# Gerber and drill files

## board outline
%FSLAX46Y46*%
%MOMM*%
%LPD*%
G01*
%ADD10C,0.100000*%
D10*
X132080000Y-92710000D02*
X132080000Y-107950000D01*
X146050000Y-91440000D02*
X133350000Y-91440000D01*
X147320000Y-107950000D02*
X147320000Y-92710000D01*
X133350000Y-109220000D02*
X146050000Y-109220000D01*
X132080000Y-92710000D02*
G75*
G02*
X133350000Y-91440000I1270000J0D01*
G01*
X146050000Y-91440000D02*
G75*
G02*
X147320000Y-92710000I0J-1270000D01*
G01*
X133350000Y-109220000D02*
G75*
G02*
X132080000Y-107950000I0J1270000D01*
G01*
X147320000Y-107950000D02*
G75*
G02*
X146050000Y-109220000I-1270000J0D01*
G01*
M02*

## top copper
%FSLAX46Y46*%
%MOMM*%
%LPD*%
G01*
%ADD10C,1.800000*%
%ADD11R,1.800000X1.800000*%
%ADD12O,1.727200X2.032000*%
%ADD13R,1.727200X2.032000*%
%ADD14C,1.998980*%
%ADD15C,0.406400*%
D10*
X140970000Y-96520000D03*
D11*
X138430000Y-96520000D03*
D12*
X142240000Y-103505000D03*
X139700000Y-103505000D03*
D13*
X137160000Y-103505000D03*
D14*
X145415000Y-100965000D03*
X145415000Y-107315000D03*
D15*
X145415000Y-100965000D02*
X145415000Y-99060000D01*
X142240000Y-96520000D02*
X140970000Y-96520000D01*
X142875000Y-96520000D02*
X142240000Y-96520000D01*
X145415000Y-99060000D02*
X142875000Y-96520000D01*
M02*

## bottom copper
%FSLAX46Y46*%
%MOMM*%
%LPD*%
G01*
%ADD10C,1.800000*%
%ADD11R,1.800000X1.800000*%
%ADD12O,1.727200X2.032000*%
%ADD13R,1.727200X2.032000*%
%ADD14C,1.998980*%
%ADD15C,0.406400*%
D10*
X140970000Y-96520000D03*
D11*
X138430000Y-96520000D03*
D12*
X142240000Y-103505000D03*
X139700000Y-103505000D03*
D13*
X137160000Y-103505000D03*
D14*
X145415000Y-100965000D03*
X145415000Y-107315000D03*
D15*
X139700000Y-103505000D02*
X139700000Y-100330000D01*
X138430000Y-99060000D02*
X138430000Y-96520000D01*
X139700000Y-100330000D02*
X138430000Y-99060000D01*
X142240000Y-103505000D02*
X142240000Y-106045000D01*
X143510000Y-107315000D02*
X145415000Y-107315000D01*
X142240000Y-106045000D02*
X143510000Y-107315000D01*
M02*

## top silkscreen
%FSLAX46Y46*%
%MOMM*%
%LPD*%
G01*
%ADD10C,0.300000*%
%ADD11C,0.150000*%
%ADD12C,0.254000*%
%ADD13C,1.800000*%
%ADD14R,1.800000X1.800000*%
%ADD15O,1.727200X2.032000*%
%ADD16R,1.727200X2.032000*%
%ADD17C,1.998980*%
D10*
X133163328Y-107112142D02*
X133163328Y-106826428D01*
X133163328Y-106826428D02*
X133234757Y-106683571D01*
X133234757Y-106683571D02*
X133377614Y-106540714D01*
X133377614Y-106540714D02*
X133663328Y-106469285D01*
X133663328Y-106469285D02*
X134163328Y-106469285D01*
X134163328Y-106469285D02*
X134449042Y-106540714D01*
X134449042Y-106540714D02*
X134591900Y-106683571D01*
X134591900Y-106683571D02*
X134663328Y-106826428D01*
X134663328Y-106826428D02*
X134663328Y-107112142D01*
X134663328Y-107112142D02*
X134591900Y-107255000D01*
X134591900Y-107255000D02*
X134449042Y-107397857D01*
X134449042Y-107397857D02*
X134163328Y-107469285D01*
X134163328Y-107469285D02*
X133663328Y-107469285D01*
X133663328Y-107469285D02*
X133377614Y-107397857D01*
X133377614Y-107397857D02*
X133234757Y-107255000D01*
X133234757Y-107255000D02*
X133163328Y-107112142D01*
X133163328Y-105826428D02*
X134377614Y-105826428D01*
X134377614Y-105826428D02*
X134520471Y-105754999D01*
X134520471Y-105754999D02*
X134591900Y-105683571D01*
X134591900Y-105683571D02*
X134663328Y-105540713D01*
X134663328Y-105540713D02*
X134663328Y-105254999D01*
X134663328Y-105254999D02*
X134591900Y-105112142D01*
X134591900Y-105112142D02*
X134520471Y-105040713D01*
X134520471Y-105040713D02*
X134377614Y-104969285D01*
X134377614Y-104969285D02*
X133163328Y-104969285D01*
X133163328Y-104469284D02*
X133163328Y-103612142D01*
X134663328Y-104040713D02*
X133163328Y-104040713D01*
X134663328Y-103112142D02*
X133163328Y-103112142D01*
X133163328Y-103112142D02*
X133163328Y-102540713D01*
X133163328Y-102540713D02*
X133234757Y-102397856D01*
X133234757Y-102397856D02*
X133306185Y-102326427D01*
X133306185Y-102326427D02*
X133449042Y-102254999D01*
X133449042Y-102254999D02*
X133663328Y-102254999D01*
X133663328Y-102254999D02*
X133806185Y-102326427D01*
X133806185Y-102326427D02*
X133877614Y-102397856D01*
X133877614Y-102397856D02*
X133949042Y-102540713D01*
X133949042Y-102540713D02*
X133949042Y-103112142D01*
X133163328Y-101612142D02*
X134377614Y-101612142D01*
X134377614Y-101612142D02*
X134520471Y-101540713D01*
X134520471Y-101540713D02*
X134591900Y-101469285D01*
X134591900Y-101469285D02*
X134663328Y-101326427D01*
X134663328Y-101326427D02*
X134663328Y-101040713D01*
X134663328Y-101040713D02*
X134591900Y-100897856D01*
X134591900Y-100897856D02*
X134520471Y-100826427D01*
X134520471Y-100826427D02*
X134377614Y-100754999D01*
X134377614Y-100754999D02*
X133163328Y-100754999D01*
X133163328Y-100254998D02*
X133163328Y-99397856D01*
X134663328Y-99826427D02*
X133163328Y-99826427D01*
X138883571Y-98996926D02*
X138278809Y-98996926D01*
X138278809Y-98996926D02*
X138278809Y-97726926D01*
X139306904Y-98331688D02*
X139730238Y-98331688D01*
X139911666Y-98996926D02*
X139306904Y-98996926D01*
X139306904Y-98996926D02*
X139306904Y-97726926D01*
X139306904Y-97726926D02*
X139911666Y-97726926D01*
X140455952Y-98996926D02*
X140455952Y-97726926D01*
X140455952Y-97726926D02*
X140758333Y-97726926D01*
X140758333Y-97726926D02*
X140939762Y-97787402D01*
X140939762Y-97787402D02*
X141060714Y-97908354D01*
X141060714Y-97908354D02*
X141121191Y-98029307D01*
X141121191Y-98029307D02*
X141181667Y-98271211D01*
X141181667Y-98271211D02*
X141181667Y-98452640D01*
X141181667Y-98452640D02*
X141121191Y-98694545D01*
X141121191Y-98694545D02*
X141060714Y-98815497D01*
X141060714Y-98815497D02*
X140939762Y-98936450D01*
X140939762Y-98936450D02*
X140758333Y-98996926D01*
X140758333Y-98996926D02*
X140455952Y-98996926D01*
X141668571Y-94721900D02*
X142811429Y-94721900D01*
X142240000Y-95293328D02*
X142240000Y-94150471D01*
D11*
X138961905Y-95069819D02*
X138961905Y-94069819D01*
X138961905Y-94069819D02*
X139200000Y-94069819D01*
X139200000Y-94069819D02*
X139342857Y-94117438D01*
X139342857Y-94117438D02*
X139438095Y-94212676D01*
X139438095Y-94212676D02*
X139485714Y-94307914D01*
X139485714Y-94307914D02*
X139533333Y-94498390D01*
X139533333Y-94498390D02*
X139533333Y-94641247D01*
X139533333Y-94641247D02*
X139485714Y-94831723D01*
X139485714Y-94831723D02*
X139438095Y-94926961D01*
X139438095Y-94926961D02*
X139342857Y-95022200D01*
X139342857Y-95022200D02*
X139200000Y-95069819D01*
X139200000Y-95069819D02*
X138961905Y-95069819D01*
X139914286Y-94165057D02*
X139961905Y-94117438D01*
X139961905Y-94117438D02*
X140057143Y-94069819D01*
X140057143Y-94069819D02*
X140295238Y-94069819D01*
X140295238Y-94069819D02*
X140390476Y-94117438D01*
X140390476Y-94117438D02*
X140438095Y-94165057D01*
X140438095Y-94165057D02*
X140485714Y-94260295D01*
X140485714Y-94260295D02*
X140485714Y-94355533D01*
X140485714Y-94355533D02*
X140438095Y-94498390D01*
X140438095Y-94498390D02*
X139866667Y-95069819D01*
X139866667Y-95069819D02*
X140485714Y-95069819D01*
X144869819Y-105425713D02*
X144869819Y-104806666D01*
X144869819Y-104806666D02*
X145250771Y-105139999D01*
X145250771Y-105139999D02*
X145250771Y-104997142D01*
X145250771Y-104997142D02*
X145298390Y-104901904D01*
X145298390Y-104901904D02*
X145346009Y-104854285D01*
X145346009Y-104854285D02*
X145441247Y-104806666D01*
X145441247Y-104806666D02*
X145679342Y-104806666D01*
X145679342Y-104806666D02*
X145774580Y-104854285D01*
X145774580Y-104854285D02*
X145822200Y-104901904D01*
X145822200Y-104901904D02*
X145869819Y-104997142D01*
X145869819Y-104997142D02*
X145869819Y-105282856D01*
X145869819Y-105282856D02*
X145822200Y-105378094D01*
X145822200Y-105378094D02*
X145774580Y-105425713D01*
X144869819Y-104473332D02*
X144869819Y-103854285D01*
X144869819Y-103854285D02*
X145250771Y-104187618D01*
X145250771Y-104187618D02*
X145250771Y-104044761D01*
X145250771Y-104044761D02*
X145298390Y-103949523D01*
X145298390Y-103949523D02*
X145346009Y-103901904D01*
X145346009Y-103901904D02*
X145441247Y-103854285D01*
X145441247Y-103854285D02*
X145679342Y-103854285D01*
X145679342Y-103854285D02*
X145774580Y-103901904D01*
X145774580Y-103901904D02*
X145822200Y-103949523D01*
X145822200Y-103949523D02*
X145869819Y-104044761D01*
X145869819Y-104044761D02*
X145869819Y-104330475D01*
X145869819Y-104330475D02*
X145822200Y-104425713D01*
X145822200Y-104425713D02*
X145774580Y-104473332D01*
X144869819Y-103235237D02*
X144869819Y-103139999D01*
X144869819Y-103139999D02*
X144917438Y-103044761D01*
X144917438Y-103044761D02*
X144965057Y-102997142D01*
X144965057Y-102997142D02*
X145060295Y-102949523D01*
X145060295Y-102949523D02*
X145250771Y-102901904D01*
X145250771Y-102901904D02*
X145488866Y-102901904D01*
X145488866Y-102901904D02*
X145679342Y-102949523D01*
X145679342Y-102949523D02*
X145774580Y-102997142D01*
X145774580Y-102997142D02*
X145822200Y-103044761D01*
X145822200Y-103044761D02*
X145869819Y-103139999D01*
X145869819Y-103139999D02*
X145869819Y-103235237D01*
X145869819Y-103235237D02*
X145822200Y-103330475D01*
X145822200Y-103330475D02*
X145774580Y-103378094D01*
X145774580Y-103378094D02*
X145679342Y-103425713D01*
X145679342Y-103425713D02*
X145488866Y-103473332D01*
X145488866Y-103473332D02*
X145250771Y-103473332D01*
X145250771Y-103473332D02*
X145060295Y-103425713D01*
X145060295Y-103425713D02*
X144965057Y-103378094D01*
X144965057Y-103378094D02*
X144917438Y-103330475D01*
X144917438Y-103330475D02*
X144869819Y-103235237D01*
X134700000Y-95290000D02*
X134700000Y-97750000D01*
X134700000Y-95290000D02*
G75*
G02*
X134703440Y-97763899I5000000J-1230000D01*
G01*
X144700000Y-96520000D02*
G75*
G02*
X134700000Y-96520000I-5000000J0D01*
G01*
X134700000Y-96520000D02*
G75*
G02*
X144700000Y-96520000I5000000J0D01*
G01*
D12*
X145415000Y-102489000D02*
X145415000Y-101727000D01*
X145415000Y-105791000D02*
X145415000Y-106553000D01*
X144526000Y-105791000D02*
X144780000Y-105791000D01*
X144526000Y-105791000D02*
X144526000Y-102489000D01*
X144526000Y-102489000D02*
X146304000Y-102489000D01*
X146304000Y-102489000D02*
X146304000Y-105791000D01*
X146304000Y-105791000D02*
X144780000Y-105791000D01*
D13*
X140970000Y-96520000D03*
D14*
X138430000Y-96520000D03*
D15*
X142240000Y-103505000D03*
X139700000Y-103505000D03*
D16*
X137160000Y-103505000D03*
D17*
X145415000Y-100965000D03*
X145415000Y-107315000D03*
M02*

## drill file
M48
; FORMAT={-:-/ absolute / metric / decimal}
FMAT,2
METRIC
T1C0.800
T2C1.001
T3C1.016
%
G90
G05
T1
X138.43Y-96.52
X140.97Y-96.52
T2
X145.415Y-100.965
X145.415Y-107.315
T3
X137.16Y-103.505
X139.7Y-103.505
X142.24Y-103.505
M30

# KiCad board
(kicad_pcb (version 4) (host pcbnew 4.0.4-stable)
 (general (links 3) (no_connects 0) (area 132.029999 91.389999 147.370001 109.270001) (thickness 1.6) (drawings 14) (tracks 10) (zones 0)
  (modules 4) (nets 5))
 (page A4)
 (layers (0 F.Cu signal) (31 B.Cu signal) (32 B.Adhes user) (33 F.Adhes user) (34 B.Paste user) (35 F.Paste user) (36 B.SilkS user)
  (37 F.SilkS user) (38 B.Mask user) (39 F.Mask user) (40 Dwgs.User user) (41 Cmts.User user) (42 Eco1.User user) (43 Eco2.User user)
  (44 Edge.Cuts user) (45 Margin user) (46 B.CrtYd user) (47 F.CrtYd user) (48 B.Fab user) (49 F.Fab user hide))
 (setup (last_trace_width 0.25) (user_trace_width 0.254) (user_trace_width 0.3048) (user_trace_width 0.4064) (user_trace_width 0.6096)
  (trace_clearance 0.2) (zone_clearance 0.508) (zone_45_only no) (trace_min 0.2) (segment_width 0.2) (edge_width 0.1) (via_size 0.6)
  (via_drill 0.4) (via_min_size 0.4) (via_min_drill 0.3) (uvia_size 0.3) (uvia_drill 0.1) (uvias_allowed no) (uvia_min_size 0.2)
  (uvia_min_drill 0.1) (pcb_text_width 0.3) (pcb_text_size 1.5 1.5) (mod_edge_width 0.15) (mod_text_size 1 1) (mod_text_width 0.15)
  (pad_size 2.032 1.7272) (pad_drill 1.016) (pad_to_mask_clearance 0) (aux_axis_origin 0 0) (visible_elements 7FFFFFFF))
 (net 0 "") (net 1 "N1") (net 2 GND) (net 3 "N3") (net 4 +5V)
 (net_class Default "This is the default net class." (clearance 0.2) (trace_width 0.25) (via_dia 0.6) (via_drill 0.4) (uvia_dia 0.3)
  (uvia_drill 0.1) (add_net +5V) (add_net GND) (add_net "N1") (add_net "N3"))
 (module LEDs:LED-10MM (layer F.Cu) (at 138.43 96.52)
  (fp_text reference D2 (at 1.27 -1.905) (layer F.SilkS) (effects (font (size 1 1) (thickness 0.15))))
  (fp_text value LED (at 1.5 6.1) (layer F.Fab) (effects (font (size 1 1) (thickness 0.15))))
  (fp_line (start -3.73 -1.23) (end -3.73 1.23) (layer F.SilkS) (width 0.15))
  (fp_arc (start 1.27 0) (end -3.73 -1.23) (angle 332.2) (layer F.SilkS) (width 0.15))
  (fp_circle (center 1.27 0) (end 1.27 5) (layer F.SilkS) (width 0.15))
  (pad 2 thru_hole circle (at 2.54 0 180) (size 1.8 1.8) (drill 0.8) (layers *.Cu *.Mask F.SilkS) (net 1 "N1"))
  (pad 1 thru_hole rect (at 0 0 180) (size 1.8 1.8) (drill 0.8) (layers *.Cu *.Mask F.SilkS) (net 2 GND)))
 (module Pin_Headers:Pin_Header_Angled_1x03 (layer F.Cu) (at 142.24 103.505 270)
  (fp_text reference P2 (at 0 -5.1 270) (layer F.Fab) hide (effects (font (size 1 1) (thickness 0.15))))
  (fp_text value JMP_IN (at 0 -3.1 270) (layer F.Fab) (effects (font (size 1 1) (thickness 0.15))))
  (pad 1 thru_hole oval (at 0 0 270) (size 2.032 1.7272) (drill 1.016) (layers *.Cu *.Mask F.SilkS) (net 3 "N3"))
  (pad 2 thru_hole oval (at 0 2.54 270) (size 2.032 1.7272) (drill 1.016) (layers *.Cu *.Mask F.SilkS) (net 2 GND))
  (pad 3 thru_hole rect (at 0 5.08 270) (size 2.032 1.7272) (drill 1.016) (layers *.Cu *.Mask F.SilkS) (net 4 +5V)))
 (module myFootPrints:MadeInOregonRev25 (layer F.Cu) (at 139.7 99.695)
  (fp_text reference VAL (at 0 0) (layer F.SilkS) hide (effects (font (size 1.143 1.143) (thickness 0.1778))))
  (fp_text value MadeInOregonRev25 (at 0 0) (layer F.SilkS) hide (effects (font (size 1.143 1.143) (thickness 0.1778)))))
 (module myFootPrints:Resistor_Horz (layer F.Cu) (at 145.415 104.14 270)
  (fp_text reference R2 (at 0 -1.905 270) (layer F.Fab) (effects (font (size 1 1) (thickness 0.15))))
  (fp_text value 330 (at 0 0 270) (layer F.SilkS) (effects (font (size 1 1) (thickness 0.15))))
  (fp_line (start -1.651 0) (end -2.413 0) (layer F.SilkS) (width 0.254))
  (fp_line (start 1.651 0) (end 2.413 0) (layer F.SilkS) (width 0.254))
  (fp_line (start 1.651 0.889) (end 1.651 0.635) (layer F.SilkS) (width 0.254))
  (fp_line (start 1.651 0.889) (end -1.651 0.889) (layer F.SilkS) (width 0.254))
  (fp_line (start -1.651 0.889) (end -1.651 -0.889) (layer F.SilkS) (width 0.254))
  (fp_line (start -1.651 -0.889) (end 1.651 -0.889) (layer F.SilkS) (width 0.254))
  (fp_line (start 1.651 -0.889) (end 1.651 0.635) (layer F.SilkS) (width 0.254))
  (pad 1 thru_hole circle (at -3.175 0 270) (size 1.99898 1.99898) (drill 1.00076) (layers *.Cu *.SilkS *.Mask) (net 1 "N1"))
  (pad 2 thru_hole circle (at 3.175 0 270) (size 1.99898 1.99898) (drill 1.00076) (layers *.Cu *.SilkS *.Mask) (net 3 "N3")))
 (gr_line (start 132.08 92.71) (end 132.08 107.95) (angle 90) (layer Edge.Cuts) (width 0.1))
 (gr_line (start 146.05 91.44) (end 133.35 91.44) (angle 90) (layer Edge.Cuts) (width 0.1))
 (gr_line (start 147.32 107.95) (end 147.32 92.71) (angle 90) (layer Edge.Cuts) (width 0.1))
 (gr_line (start 133.35 109.22) (end 146.05 109.22) (angle 90) (layer Edge.Cuts) (width 0.1))
 (gr_arc (start 133.35 92.71) (end 132.08 92.71) (angle 90) (layer Edge.Cuts) (width 0.1))
 (gr_arc (start 146.05 92.71) (end 146.05 91.44) (angle 90) (layer Edge.Cuts) (width 0.1))
 (gr_arc (start 133.35 107.95) (end 133.35 109.22) (angle 90) (layer Edge.Cuts) (width 0.1))
 (gr_arc (start 146.05 107.95) (end 147.32 107.95) (angle 90) (layer Edge.Cuts) (width 0.1))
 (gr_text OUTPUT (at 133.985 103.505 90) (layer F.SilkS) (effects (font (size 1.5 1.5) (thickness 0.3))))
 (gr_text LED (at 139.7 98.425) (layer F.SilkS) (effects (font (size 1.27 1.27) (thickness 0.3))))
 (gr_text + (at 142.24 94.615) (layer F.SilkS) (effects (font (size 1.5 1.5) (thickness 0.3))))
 (segment (start 139.7 103.505) (end 139.7 100.33) (width 0.4064) (layer B.Cu) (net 2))
 (segment (start 138.43 99.06) (end 138.43 96.52) (width 0.4064) (layer B.Cu) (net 2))
 (segment (start 139.7 100.33) (end 138.43 99.06) (width 0.4064) (layer B.Cu) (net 2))
 (segment (start 145.415 100.965) (end 145.415 99.06) (width 0.4064) (layer F.Cu) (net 1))
 (segment (start 142.24 96.52) (end 140.97 96.52) (width 0.4064) (layer F.Cu) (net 1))
 (segment (start 142.875 96.52) (end 142.24 96.52) (width 0.4064) (layer F.Cu) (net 1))
 (segment (start 145.415 99.06) (end 142.875 96.52) (width 0.4064) (layer F.Cu) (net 1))
 (segment (start 142.24 103.505) (end 142.24 106.045) (width 0.4064) (layer B.Cu) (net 3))
 (segment (start 143.51 107.315) (end 145.415 107.315) (width 0.4064) (layer B.Cu) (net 3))
 (segment (start 142.24 106.045) (end 143.51 107.315) (width 0.4064) (layer B.Cu) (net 3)))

